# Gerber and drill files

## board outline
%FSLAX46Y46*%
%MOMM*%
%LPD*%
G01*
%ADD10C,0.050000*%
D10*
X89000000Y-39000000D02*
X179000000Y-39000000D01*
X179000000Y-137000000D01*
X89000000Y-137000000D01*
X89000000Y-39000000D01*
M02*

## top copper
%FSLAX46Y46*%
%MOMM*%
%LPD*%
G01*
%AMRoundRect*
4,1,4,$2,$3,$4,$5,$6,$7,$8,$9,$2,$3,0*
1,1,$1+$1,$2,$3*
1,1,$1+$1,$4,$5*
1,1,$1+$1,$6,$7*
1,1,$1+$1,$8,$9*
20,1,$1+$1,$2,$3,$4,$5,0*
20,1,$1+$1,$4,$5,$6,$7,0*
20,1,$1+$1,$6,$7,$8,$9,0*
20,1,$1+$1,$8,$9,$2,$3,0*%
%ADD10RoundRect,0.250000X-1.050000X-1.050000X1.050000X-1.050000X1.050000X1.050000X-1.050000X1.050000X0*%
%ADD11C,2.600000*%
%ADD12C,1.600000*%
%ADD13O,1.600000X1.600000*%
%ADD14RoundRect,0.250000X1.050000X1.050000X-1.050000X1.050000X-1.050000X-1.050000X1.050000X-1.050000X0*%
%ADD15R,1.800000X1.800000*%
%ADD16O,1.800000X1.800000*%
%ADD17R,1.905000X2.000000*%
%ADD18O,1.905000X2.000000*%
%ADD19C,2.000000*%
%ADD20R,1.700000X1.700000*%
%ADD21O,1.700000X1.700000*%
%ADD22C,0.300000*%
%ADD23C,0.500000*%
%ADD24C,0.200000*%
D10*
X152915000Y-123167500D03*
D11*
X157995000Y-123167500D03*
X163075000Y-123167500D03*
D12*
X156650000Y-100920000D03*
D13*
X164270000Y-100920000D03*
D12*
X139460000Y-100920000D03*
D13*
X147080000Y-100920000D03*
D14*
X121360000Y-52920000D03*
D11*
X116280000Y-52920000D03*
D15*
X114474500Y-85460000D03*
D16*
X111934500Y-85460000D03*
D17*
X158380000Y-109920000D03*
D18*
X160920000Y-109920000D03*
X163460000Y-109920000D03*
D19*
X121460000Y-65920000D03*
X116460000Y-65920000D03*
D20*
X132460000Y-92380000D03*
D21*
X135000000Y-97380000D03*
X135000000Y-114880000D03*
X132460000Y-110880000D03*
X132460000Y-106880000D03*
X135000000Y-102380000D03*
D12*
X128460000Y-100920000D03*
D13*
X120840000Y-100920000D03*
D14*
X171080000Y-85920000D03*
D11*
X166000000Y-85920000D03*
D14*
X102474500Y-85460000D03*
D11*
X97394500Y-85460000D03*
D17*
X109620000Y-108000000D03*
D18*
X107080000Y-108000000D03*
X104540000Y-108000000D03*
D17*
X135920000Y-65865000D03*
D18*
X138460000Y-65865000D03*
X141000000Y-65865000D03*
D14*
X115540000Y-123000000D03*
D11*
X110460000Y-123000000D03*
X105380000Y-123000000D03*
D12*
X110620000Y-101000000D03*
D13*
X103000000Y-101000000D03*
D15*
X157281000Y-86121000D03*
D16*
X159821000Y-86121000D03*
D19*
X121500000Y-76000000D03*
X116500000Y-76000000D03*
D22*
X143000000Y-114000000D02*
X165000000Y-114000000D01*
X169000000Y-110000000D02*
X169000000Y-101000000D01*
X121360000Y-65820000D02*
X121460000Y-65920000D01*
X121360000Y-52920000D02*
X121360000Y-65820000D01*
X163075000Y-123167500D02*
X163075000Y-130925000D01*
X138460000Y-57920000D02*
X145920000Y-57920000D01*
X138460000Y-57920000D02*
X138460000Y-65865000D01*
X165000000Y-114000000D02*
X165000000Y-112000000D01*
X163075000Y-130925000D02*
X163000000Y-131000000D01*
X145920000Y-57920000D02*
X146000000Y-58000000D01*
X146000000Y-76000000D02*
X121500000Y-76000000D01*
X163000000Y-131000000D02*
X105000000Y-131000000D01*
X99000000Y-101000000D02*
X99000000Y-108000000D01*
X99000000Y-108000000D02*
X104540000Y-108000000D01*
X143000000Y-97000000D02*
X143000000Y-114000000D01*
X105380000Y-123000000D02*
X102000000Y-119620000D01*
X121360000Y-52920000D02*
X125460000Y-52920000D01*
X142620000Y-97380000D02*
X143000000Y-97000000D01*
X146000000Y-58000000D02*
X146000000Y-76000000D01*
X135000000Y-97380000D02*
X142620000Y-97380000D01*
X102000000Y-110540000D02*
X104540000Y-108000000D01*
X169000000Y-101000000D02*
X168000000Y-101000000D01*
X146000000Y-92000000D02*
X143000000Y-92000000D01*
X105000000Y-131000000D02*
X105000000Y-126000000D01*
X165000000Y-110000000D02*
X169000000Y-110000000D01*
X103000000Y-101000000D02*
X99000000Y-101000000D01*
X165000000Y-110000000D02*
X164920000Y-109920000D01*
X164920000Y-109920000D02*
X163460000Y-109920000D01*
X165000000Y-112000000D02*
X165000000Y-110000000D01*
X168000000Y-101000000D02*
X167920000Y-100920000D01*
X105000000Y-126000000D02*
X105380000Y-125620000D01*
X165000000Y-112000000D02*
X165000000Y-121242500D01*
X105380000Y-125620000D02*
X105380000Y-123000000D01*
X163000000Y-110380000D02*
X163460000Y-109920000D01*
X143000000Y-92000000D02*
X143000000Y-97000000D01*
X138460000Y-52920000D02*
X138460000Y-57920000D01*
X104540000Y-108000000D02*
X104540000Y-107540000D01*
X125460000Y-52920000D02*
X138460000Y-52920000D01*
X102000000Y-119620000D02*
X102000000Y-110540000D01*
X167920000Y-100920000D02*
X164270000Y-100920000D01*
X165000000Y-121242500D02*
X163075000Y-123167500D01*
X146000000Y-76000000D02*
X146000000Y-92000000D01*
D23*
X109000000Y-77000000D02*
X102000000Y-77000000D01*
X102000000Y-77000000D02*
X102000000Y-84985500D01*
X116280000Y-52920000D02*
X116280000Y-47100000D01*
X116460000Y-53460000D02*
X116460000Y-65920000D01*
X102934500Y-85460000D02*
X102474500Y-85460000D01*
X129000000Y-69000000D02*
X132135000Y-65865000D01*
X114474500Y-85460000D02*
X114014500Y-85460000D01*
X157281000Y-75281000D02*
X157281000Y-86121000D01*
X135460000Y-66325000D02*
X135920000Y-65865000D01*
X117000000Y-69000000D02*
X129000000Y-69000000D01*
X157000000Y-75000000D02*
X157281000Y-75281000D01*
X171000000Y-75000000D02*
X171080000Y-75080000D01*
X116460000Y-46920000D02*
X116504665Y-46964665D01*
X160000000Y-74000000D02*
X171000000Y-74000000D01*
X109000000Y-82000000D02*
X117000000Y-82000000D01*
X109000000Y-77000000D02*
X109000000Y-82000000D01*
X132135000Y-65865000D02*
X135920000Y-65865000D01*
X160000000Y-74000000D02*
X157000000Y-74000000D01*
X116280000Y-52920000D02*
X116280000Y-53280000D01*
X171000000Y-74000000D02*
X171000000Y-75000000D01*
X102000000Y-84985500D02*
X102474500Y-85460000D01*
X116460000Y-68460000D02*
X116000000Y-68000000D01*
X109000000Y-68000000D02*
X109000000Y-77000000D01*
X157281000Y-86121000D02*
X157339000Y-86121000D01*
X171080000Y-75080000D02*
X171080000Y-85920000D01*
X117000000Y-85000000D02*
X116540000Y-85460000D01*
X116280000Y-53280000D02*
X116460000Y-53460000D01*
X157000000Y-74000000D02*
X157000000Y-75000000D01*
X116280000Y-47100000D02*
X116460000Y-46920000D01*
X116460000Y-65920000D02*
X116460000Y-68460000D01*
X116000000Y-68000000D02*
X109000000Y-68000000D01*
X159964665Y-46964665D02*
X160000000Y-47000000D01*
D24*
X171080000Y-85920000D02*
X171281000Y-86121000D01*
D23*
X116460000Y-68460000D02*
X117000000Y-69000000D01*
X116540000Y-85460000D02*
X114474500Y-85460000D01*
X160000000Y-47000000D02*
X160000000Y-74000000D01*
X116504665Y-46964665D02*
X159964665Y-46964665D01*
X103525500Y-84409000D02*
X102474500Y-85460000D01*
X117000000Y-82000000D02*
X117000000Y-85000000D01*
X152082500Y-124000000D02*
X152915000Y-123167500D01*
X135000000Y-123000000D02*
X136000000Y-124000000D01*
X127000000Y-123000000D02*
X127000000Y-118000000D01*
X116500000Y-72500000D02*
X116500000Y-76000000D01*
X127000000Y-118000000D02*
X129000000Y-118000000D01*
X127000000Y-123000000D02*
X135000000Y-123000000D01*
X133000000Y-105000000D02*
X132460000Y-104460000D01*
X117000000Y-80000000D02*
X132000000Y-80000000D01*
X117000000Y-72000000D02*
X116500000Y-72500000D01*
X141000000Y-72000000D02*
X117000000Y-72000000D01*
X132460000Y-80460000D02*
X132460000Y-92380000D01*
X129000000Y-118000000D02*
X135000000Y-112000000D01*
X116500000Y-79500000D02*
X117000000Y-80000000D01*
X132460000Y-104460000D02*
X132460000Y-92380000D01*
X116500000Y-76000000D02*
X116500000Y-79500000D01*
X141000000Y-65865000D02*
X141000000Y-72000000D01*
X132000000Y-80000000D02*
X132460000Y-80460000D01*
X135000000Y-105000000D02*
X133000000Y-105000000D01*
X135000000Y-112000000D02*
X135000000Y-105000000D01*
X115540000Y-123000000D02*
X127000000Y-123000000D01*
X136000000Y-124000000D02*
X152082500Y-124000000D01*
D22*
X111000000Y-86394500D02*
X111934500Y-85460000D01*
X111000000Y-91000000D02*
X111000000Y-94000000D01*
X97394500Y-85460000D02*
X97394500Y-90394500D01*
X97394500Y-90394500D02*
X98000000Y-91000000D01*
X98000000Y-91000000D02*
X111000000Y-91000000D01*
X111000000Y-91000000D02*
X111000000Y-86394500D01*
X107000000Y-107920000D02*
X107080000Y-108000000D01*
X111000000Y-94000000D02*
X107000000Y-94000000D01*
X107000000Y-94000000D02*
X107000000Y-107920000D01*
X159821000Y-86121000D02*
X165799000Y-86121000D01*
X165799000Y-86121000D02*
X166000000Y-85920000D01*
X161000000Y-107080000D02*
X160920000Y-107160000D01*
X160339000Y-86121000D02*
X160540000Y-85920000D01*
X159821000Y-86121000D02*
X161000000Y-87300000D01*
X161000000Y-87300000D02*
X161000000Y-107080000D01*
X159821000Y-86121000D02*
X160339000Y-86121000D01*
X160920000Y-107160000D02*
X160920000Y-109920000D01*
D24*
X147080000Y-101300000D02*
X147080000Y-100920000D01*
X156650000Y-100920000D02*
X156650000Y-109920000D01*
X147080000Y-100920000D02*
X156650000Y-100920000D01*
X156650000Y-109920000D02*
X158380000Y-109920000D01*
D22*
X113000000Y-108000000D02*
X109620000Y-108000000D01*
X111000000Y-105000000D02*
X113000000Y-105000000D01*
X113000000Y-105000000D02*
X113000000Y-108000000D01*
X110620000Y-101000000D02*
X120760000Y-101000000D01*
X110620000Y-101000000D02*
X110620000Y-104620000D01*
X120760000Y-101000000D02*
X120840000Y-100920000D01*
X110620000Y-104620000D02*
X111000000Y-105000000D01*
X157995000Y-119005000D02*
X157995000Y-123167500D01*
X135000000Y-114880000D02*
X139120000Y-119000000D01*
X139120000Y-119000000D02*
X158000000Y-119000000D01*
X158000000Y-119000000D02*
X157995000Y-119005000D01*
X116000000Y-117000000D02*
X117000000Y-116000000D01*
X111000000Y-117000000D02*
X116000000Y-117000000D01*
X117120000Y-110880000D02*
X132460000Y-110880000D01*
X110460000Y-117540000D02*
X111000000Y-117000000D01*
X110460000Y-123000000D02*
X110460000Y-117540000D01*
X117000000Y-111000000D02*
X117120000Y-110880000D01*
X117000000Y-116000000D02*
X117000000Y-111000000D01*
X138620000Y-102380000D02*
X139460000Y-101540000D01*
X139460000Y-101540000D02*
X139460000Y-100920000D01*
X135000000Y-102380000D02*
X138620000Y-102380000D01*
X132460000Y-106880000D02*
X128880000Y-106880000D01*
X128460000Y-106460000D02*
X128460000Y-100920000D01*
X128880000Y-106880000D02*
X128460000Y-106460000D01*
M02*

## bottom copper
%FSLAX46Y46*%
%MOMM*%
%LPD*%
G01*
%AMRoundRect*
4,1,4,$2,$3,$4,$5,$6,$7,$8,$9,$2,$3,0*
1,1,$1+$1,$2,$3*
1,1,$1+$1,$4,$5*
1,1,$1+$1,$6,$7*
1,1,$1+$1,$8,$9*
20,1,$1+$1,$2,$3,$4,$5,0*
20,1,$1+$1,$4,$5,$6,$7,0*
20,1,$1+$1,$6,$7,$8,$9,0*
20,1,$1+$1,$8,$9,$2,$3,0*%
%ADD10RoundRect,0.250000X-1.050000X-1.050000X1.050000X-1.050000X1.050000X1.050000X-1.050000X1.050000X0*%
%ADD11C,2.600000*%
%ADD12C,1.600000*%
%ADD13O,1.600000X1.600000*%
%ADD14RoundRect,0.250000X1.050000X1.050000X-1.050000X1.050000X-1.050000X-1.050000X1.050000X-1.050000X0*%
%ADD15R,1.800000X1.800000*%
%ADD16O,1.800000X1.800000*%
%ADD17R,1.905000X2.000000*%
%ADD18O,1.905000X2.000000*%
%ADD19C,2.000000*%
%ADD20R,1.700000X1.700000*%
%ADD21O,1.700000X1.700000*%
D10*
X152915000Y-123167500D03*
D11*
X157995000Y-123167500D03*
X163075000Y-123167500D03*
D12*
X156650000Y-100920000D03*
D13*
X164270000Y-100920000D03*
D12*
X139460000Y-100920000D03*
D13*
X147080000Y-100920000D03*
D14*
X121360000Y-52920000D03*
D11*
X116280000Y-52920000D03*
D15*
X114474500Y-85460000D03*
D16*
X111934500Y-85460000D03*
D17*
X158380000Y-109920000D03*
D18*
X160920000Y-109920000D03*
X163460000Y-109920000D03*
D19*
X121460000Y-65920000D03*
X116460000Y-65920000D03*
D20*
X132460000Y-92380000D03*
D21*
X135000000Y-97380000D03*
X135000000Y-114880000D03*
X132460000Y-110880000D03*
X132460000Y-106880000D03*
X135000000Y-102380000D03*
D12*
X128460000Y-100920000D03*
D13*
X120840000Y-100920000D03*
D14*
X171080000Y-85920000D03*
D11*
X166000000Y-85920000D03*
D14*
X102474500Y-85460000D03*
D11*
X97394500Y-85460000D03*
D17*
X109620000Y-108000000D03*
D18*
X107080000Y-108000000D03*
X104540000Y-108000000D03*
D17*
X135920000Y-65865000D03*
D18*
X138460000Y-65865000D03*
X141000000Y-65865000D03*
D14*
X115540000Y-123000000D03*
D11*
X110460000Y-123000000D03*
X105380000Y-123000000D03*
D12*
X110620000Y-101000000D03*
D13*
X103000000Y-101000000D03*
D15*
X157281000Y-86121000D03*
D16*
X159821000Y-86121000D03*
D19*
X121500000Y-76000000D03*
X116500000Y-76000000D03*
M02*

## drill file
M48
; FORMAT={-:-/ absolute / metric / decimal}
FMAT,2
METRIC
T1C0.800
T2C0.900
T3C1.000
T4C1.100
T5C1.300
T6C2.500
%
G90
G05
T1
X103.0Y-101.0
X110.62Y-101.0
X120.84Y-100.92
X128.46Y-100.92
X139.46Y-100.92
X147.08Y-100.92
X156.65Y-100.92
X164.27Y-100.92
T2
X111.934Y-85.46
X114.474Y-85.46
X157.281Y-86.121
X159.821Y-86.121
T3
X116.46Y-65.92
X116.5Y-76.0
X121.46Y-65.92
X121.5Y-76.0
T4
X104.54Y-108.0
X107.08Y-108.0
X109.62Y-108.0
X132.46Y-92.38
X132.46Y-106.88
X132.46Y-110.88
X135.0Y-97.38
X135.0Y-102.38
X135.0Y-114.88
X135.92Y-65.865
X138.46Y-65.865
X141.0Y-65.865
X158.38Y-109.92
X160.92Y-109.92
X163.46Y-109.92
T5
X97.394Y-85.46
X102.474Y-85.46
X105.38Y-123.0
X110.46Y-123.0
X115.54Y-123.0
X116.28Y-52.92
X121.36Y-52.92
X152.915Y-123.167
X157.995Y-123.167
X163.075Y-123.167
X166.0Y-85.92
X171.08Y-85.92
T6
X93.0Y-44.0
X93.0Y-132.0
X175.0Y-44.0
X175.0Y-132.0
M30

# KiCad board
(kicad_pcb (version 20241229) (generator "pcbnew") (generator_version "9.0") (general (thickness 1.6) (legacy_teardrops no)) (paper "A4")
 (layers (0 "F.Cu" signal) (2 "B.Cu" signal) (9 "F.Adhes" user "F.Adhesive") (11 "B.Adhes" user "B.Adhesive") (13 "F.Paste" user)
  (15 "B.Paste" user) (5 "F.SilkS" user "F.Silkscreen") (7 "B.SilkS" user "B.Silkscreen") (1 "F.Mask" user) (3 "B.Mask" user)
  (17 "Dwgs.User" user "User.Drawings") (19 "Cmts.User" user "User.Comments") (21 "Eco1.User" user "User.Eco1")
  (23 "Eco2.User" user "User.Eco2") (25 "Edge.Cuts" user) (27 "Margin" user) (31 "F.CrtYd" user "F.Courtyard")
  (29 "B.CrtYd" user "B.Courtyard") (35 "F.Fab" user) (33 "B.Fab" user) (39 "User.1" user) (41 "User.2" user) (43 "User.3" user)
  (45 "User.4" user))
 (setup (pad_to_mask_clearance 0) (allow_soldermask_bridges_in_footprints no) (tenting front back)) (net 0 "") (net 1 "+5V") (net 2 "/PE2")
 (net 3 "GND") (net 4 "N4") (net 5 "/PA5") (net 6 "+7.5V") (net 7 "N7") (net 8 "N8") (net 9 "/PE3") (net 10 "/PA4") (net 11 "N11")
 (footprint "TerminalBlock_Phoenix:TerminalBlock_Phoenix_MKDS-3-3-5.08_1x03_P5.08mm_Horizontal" (layer "F.Cu") (at 152.915 123.1675)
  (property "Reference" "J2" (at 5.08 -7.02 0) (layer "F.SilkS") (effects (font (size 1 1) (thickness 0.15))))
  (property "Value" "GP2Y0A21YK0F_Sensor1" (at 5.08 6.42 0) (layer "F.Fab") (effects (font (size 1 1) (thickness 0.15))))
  (pad "1" thru_hole roundrect (at 0 0) (size 2.6 2.6) (drill 1.3) (layers "*.Cu" "*.Mask") (remove_unused_layers no)
   (roundrect_rratio 0.096154) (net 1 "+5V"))
  (pad "2" thru_hole circle (at 5.08 0) (size 2.6 2.6) (drill 1.3) (layers "*.Cu" "*.Mask") (remove_unused_layers no) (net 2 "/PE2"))
  (pad "3" thru_hole circle (at 10.16 0) (size 2.6 2.6) (drill 1.3) (layers "*.Cu" "*.Mask") (remove_unused_layers no) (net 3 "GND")))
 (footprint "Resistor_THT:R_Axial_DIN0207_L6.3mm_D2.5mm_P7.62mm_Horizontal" (layer "F.Cu") (at 156.65 100.92)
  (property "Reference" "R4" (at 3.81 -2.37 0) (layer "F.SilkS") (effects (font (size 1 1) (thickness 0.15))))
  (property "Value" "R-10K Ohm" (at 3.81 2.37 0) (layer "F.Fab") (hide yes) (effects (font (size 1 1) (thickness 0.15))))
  (pad "1" thru_hole circle (at 0 0) (size 1.6 1.6) (drill 0.8) (layers "*.Cu" "*.Mask") (remove_unused_layers no) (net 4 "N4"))
  (pad "2" thru_hole oval (at 7.62 0) (size 1.6 1.6) (drill 0.8) (layers "*.Cu" "*.Mask") (remove_unused_layers no) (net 3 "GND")))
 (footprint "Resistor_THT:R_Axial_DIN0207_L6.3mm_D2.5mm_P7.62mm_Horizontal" (layer "F.Cu") (at 139.46 100.92)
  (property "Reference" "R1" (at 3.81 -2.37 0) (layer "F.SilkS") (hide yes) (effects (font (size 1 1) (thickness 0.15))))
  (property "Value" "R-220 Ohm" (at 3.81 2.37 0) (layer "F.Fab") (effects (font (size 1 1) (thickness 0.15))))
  (pad "1" thru_hole circle (at 0 0) (size 1.6 1.6) (drill 0.8) (layers "*.Cu" "*.Mask") (remove_unused_layers no) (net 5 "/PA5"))
  (pad "2" thru_hole oval (at 7.62 0) (size 1.6 1.6) (drill 0.8) (layers "*.Cu" "*.Mask") (remove_unused_layers no) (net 4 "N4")))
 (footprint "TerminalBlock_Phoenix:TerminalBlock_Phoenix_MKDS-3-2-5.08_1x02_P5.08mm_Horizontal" (layer "F.Cu") (at 121.36 52.92 180)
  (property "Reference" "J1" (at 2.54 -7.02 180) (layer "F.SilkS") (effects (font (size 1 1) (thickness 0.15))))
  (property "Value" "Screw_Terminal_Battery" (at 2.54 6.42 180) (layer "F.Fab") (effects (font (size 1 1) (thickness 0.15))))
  (pad "1" thru_hole roundrect (at 0 0 180) (size 2.6 2.6) (drill 1.3) (layers "*.Cu" "*.Mask") (remove_unused_layers no)
   (roundrect_rratio 0.096154) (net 3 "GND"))
  (pad "2" thru_hole circle (at 5.08 0 180) (size 2.6 2.6) (drill 1.3) (layers "*.Cu" "*.Mask") (remove_unused_layers no) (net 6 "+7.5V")))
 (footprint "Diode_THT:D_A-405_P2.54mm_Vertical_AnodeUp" (layer "F.Cu") (at 114.4745 85.46 180)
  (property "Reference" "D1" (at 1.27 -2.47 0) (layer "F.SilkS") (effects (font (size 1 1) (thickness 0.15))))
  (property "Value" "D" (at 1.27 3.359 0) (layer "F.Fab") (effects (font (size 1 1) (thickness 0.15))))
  (pad "1" thru_hole rect (at 0 0 180) (size 1.8 1.8) (drill 0.9) (layers "*.Cu" "*.Mask") (remove_unused_layers no) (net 6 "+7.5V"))
  (pad "2" thru_hole oval (at 2.54 0 180) (size 1.8 1.8) (drill 0.9) (layers "*.Cu" "*.Mask") (remove_unused_layers no) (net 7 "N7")))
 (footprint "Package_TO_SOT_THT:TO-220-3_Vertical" (layer "F.Cu") (at 158.38 109.92)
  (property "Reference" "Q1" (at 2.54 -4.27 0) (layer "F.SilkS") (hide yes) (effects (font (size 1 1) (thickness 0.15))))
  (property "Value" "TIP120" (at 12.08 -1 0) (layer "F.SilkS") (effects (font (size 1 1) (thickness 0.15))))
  (pad "1" thru_hole rect (at 0 0) (size 1.905 2) (drill 1.1) (layers "*.Cu" "*.Mask") (remove_unused_layers no) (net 4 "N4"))
  (pad "2" thru_hole oval (at 2.54 0) (size 1.905 2) (drill 1.1) (layers "*.Cu" "*.Mask") (remove_unused_layers no) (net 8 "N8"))
  (pad "3" thru_hole oval (at 5.08 0) (size 1.905 2) (drill 1.1) (layers "*.Cu" "*.Mask") (remove_unused_layers no) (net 3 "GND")))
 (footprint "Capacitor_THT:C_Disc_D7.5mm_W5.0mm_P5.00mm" (layer "F.Cu") (at 121.46 65.92 180)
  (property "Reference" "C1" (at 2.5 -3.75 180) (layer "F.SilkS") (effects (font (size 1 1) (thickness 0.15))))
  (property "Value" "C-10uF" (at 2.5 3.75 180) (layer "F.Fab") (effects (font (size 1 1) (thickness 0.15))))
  (pad "1" thru_hole circle (at 0 0 180) (size 2 2) (drill 1) (layers "*.Cu" "*.Mask") (remove_unused_layers no) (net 3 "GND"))
  (pad "2" thru_hole circle (at 5 0 180) (size 2 2) (drill 1) (layers "*.Cu" "*.Mask") (remove_unused_layers no) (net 6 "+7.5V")))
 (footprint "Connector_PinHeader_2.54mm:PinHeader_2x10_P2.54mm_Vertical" (layer "F.Cu") (at 132.46 92.38)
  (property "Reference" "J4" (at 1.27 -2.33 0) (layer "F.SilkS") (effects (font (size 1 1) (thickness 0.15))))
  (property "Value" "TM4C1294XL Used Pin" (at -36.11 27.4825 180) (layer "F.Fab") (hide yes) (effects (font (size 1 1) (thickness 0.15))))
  (pad "1" thru_hole rect (at 0 0) (size 1.7 1.7) (drill 1.1) (layers "*.Cu" "*.Mask") (remove_unused_layers no) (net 1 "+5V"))
  (pad "2" thru_hole oval (at 2.54 5) (size 1.7 1.7) (drill 1.1) (layers "*.Cu" "*.Mask") (remove_unused_layers no) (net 3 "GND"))
  (pad "4" thru_hole oval (at 2.54 22.5) (size 1.7 1.7) (drill 1.1) (layers "*.Cu" "*.Mask") (remove_unused_layers no) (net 2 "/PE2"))
  (pad "5" thru_hole oval (at 0 18.5) (size 1.7 1.7) (drill 1.1) (layers "*.Cu" "*.Mask") (remove_unused_layers no) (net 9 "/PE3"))
  (pad "7" thru_hole oval (at 0 14.5) (size 1.7 1.7) (drill 1.1) (layers "*.Cu" "*.Mask") (remove_unused_layers no) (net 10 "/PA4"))
  (pad "8" thru_hole oval (at 2.54 10) (size 1.7 1.7) (drill 1.1) (layers "*.Cu" "*.Mask") (remove_unused_layers no) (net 5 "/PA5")))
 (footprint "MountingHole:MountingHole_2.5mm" (layer "F.Cu") (at 93 44)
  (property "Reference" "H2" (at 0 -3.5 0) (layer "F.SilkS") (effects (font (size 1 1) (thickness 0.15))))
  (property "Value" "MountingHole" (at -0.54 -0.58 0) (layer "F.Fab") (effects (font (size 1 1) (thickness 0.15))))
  (pad "" np_thru_hole circle (at 0 0) (size 2.5 2.5) (drill 2.5) (layers "*.Cu" "*.Mask")))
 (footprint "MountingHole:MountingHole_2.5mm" (layer "F.Cu") (at 93 132)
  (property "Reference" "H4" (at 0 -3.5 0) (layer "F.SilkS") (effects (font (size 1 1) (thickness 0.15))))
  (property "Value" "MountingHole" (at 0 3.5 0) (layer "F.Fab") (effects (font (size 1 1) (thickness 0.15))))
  (pad "" np_thru_hole circle (at 0 0) (size 2.5 2.5) (drill 2.5) (layers "*.Cu" "*.Mask")))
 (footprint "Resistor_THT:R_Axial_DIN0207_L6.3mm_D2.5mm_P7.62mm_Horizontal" (layer "F.Cu") (at 128.46 100.92 180)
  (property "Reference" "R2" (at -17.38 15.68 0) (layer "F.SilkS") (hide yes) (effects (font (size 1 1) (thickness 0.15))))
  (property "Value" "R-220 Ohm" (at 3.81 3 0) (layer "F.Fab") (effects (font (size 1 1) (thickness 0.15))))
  (pad "1" thru_hole circle (at 0 0 180) (size 1.6 1.6) (drill 0.8) (layers "*.Cu" "*.Mask") (remove_unused_layers no) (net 10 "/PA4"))
  (pad "2" thru_hole oval (at 7.62 0 180) (size 1.6 1.6) (drill 0.8) (layers "*.Cu" "*.Mask") (remove_unused_layers no) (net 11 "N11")))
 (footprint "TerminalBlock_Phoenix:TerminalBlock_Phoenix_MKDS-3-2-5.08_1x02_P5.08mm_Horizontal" (layer "F.Cu") (at 171.08 85.92 180)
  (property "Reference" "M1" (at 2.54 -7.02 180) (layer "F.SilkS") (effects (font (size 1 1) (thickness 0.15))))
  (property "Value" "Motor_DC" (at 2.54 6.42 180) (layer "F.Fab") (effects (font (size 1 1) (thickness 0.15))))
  (pad "1" thru_hole roundrect (at 0 0 180) (size 2.6 2.6) (drill 1.3) (layers "*.Cu" "*.Mask") (remove_unused_layers no)
   (roundrect_rratio 0.096154) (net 6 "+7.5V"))
  (pad "2" thru_hole circle (at 5.08 0 180) (size 2.6 2.6) (drill 1.3) (layers "*.Cu" "*.Mask") (remove_unused_layers no) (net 8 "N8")))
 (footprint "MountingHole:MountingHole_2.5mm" (layer "F.Cu") (at 175 132)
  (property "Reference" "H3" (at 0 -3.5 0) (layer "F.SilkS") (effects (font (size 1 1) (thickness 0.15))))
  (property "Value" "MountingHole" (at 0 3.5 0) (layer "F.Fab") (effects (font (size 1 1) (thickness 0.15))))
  (pad "" np_thru_hole circle (at 0 0) (size 2.5 2.5) (drill 2.5) (layers "*.Cu" "*.Mask")))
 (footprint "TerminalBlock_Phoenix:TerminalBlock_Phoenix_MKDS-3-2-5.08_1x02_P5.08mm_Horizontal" (layer "F.Cu") (at 102.4745 85.46 180)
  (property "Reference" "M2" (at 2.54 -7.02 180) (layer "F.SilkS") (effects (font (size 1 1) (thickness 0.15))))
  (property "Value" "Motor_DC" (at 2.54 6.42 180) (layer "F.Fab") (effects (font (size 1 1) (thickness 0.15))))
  (pad "1" thru_hole roundrect (at 0 0 180) (size 2.6 2.6) (drill 1.3) (layers "*.Cu" "*.Mask") (remove_unused_layers no)
   (roundrect_rratio 0.096154) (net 6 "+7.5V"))
  (pad "2" thru_hole circle (at 5.08 0 180) (size 2.6 2.6) (drill 1.3) (layers "*.Cu" "*.Mask") (remove_unused_layers no) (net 7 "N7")))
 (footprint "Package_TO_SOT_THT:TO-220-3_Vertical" (layer "F.Cu") (at 109.62 108 180)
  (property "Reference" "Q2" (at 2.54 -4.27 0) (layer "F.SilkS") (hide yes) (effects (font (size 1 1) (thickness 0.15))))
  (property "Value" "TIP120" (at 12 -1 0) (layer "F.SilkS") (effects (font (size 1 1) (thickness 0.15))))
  (pad "1" thru_hole rect (at 0 0 180) (size 1.905 2) (drill 1.1) (layers "*.Cu" "*.Mask") (remove_unused_layers no) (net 11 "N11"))
  (pad "2" thru_hole oval (at 2.54 0 180) (size 1.905 2) (drill 1.1) (layers "*.Cu" "*.Mask") (remove_unused_layers no) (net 7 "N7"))
  (pad "3" thru_hole oval (at 5.08 0 180) (size 1.905 2) (drill 1.1) (layers "*.Cu" "*.Mask") (remove_unused_layers no) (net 3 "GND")))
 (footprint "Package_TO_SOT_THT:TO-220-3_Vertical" (layer "F.Cu") (at 135.92 65.865)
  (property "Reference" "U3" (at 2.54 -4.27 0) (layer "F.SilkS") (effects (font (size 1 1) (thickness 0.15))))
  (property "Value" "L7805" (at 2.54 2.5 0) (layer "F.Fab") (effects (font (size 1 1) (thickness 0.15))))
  (pad "1" thru_hole rect (at 0 0) (size 1.905 2) (drill 1.1) (layers "*.Cu" "*.Mask") (remove_unused_layers no) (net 6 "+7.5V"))
  (pad "2" thru_hole oval (at 2.54 0) (size 1.905 2) (drill 1.1) (layers "*.Cu" "*.Mask") (remove_unused_layers no) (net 3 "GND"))
  (pad "3" thru_hole oval (at 5.08 0) (size 1.905 2) (drill 1.1) (layers "*.Cu" "*.Mask") (remove_unused_layers no) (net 1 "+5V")))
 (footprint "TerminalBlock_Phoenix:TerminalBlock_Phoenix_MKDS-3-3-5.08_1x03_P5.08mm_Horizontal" (layer "F.Cu") (at 115.54 123 180)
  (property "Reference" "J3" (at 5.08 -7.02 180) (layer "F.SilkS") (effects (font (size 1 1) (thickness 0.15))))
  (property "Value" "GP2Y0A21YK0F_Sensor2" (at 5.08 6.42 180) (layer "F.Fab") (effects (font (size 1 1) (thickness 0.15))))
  (pad "1" thru_hole roundrect (at 0 0 180) (size 2.6 2.6) (drill 1.3) (layers "*.Cu" "*.Mask") (remove_unused_layers no)
   (roundrect_rratio 0.096154) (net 1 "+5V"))
  (pad "2" thru_hole circle (at 5.08 0 180) (size 2.6 2.6) (drill 1.3) (layers "*.Cu" "*.Mask") (remove_unused_layers no) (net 9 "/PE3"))
  (pad "3" thru_hole circle (at 10.16 0 180) (size 2.6 2.6) (drill 1.3) (layers "*.Cu" "*.Mask") (remove_unused_layers no) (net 3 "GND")))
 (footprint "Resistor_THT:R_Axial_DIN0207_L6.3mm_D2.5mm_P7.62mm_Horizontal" (layer "F.Cu") (at 110.62 101 180)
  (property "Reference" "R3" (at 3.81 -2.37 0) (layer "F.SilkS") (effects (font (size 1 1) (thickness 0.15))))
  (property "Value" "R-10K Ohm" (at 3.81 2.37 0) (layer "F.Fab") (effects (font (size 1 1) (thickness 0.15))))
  (pad "1" thru_hole circle (at 0 0 180) (size 1.6 1.6) (drill 0.8) (layers "*.Cu" "*.Mask") (remove_unused_layers no) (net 11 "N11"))
  (pad "2" thru_hole oval (at 7.62 0 180) (size 1.6 1.6) (drill 0.8) (layers "*.Cu" "*.Mask") (remove_unused_layers no) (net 3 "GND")))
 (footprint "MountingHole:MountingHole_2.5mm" (layer "F.Cu") (at 175 44)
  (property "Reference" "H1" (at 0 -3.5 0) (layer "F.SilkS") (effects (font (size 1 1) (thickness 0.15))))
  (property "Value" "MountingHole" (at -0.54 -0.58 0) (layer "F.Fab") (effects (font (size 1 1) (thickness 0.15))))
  (pad "" np_thru_hole circle (at 0 0) (size 2.5 2.5) (drill 2.5) (layers "*.Cu" "*.Mask")))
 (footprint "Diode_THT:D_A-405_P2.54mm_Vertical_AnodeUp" (layer "F.Cu") (at 157.281 86.121)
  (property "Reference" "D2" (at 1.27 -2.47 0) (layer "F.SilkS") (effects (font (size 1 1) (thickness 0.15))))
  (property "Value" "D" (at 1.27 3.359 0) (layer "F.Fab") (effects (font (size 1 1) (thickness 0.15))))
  (pad "1" thru_hole rect (at 0 0) (size 1.8 1.8) (drill 0.9) (layers "*.Cu" "*.Mask") (remove_unused_layers no) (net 6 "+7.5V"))
  (pad "2" thru_hole oval (at 2.54 0) (size 1.8 1.8) (drill 0.9) (layers "*.Cu" "*.Mask") (remove_unused_layers no) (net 8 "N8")))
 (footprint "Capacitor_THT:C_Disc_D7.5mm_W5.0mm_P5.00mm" (layer "F.Cu") (at 121.5 76 180)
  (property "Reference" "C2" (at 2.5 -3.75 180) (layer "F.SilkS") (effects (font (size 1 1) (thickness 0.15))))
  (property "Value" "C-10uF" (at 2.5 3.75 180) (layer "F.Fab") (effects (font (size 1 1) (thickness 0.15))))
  (pad "1" thru_hole circle (at 0 0 180) (size 2 2) (drill 1) (layers "*.Cu" "*.Mask") (remove_unused_layers no) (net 3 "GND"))
  (pad "2" thru_hole circle (at 5 0 180) (size 2 2) (drill 1) (layers "*.Cu" "*.Mask") (remove_unused_layers no) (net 1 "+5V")))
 (gr_rect (start 89 39) (end 179 137) (stroke (width 0.05) (type default)) (fill no) (layer "Edge.Cuts"))
 (segment (start 143 114) (end 165 114) (width 0.3) (layer "F.Cu") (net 3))
 (segment (start 169 110) (end 169 101) (width 0.3) (layer "F.Cu") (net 3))
 (segment (start 121.36 65.82) (end 121.46 65.92) (width 0.3) (layer "F.Cu") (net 3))
 (segment (start 121.36 52.92) (end 121.36 65.82) (width 0.3) (layer "F.Cu") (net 3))
 (segment (start 163.075 123.1675) (end 163.075 130.925) (width 0.3) (layer "F.Cu") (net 3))
 (segment (start 138.46 57.92) (end 145.92 57.92) (width 0.3) (layer "F.Cu") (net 3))
 (segment (start 138.46 57.92) (end 138.46 65.865) (width 0.3) (layer "F.Cu") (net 3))
 (segment (start 165 114) (end 165 112) (width 0.3) (layer "F.Cu") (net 3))
 (segment (start 163.075 130.925) (end 163 131) (width 0.3) (layer "F.Cu") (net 3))
 (segment (start 145.92 57.92) (end 146 58) (width 0.3) (layer "F.Cu") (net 3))
 (segment (start 146 76) (end 121.5 76) (width 0.3) (layer "F.Cu") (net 3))
 (segment (start 163 131) (end 105 131) (width 0.3) (layer "F.Cu") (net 3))
 (segment (start 99 101) (end 99 108) (width 0.3) (layer "F.Cu") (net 3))
 (segment (start 99 108) (end 104.54 108) (width 0.3) (layer "F.Cu") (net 3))
 (segment (start 143 97) (end 143 114) (width 0.3) (layer "F.Cu") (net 3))
 (segment (start 105.38 123) (end 102 119.62) (width 0.3) (layer "F.Cu") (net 3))
 (segment (start 121.36 52.92) (end 125.46 52.92) (width 0.3) (layer "F.Cu") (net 3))
 (segment (start 142.62 97.38) (end 143 97) (width 0.3) (layer "F.Cu") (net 3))
 (segment (start 146 58) (end 146 76) (width 0.3) (layer "F.Cu") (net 3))
 (segment (start 135 97.38) (end 142.62 97.38) (width 0.3) (layer "F.Cu") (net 3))
 (segment (start 102 110.54) (end 104.54 108) (width 0.3) (layer "F.Cu") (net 3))
 (segment (start 169 101) (end 168 101) (width 0.3) (layer "F.Cu") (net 3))
 (segment (start 146 92) (end 143 92) (width 0.3) (layer "F.Cu") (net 3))
 (segment (start 105 131) (end 105 126) (width 0.3) (layer "F.Cu") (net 3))
 (segment (start 165 110) (end 169 110) (width 0.3) (layer "F.Cu") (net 3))
 (segment (start 103 101) (end 99 101) (width 0.3) (layer "F.Cu") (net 3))
 (segment (start 165 110) (end 164.92 109.92) (width 0.3) (layer "F.Cu") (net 3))
 (segment (start 164.92 109.92) (end 163.46 109.92) (width 0.3) (layer "F.Cu") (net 3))
 (segment (start 165 112) (end 165 110) (width 0.3) (layer "F.Cu") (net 3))
 (segment (start 168 101) (end 167.92 100.92) (width 0.3) (layer "F.Cu") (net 3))
 (segment (start 105 126) (end 105.38 125.62) (width 0.3) (layer "F.Cu") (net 3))
 (segment (start 165 112) (end 165 121.2425) (width 0.3) (layer "F.Cu") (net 3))
 (segment (start 105.38 125.62) (end 105.38 123) (width 0.3) (layer "F.Cu") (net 3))
 (segment (start 163 110.38) (end 163.46 109.92) (width 0.3) (layer "F.Cu") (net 3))
 (segment (start 143 92) (end 143 97) (width 0.3) (layer "F.Cu") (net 3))
 (segment (start 138.46 52.92) (end 138.46 57.92) (width 0.3) (layer "F.Cu") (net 3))
 (segment (start 104.54 108) (end 104.54 107.54) (width 0.3) (layer "F.Cu") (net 3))
 (segment (start 125.46 52.92) (end 138.46 52.92) (width 0.3) (layer "F.Cu") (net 3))
 (segment (start 102 119.62) (end 102 110.54) (width 0.3) (layer "F.Cu") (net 3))
 (segment (start 167.92 100.92) (end 164.27 100.92) (width 0.3) (layer "F.Cu") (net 3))
 (segment (start 165 121.2425) (end 163.075 123.1675) (width 0.3) (layer "F.Cu") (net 3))
 (segment (start 146 76) (end 146 92) (width 0.3) (layer "F.Cu") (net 3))
 (segment (start 109 77) (end 102 77) (width 0.5) (layer "F.Cu") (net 6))
 (segment (start 102 77) (end 102 84.9855) (width 0.5) (layer "F.Cu") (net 6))
 (segment (start 116.28 52.92) (end 116.28 47.1) (width 0.5) (layer "F.Cu") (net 6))
 (segment (start 116.46 53.46) (end 116.46 65.92) (width 0.5) (layer "F.Cu") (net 6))
 (segment (start 102.9345 85.46) (end 102.4745 85.46) (width 0.5) (layer "F.Cu") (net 6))
 (segment (start 129 69) (end 132.135 65.865) (width 0.5) (layer "F.Cu") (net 6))
 (segment (start 114.4745 85.46) (end 114.0145 85.46) (width 0.5) (layer "F.Cu") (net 6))
 (segment (start 157.281 75.281) (end 157.281 86.121) (width 0.5) (layer "F.Cu") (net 6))
 (segment (start 135.46 66.325) (end 135.92 65.865) (width 0.5) (layer "F.Cu") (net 6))
 (segment (start 117 69) (end 129 69) (width 0.5) (layer "F.Cu") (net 6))
 (segment (start 157 75) (end 157.281 75.281) (width 0.5) (layer "F.Cu") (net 6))
 (segment (start 171 75) (end 171.08 75.08) (width 0.5) (layer "F.Cu") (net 6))
 (segment (start 116.46 46.92) (end 116.504665 46.964665) (width 0.5) (layer "F.Cu") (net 6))
 (segment (start 160 74) (end 171 74) (width 0.5) (layer "F.Cu") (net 6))
 (segment (start 109 82) (end 117 82) (width 0.5) (layer "F.Cu") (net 6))
 (segment (start 109 77) (end 109 82) (width 0.5) (layer "F.Cu") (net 6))
 (segment (start 132.135 65.865) (end 135.92 65.865) (width 0.5) (layer "F.Cu") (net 6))
 (segment (start 160 74) (end 157 74) (width 0.5) (layer "F.Cu") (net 6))
 (segment (start 116.28 52.92) (end 116.28 53.28) (width 0.5) (layer "F.Cu") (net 6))
 (segment (start 171 74) (end 171 75) (width 0.5) (layer "F.Cu") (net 6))
 (segment (start 102 84.9855) (end 102.4745 85.46) (width 0.5) (layer "F.Cu") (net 6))
 (segment (start 116.46 68.46) (end 116 68) (width 0.5) (layer "F.Cu") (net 6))
 (segment (start 109 68) (end 109 77) (width 0.5) (layer "F.Cu") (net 6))
 (segment (start 157.281 86.121) (end 157.339 86.121) (width 0.5) (layer "F.Cu") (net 6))
 (segment (start 171.08 75.08) (end 171.08 85.92) (width 0.5) (layer "F.Cu") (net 6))
 (segment (start 117 85) (end 116.54 85.46) (width 0.5) (layer "F.Cu") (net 6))
 (segment (start 116.28 53.28) (end 116.46 53.46) (width 0.5) (layer "F.Cu") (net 6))
 (segment (start 157 74) (end 157 75) (width 0.5) (layer "F.Cu") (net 6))
 (segment (start 116.28 47.1) (end 116.46 46.92) (width 0.5) (layer "F.Cu") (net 6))
 (segment (start 116.46 65.92) (end 116.46 68.46) (width 0.5) (layer "F.Cu") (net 6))
 (segment (start 116 68) (end 109 68) (width 0.5) (layer "F.Cu") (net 6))
 (segment (start 159.964665 46.964665) (end 160 47) (width 0.5) (layer "F.Cu") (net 6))
 (segment (start 171.08 85.92) (end 171.281 86.121) (width 0.2) (layer "F.Cu") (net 6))
 (segment (start 116.46 68.46) (end 117 69) (width 0.5) (layer "F.Cu") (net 6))
 (segment (start 116.54 85.46) (end 114.4745 85.46) (width 0.5) (layer "F.Cu") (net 6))
 (segment (start 160 47) (end 160 74) (width 0.5) (layer "F.Cu") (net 6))
 (segment (start 116.504665 46.964665) (end 159.964665 46.964665) (width 0.5) (layer "F.Cu") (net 6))
 (segment (start 103.5255 84.409) (end 102.4745 85.46) (width 0.5) (layer "F.Cu") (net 6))
 (segment (start 117 82) (end 117 85) (width 0.5) (layer "F.Cu") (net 6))
 (segment (start 152.0825 124) (end 152.915 123.1675) (width 0.5) (layer "F.Cu") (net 1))
 (segment (start 135 123) (end 136 124) (width 0.5) (layer "F.Cu") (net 1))
 (segment (start 127 123) (end 127 118) (width 0.5) (layer "F.Cu") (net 1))
 (segment (start 116.5 72.5) (end 116.5 76) (width 0.5) (layer "F.Cu") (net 1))
 (segment (start 127 118) (end 129 118) (width 0.5) (layer "F.Cu") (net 1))
 (segment (start 127 123) (end 135 123) (width 0.5) (layer "F.Cu") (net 1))
 (segment (start 133 105) (end 132.46 104.46) (width 0.5) (layer "F.Cu") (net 1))
 (segment (start 117 80) (end 132 80) (width 0.5) (layer "F.Cu") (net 1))
 (segment (start 117 72) (end 116.5 72.5) (width 0.5) (layer "F.Cu") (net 1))
 (segment (start 141 72) (end 117 72) (width 0.5) (layer "F.Cu") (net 1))
 (segment (start 132.46 80.46) (end 132.46 92.38) (width 0.5) (layer "F.Cu") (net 1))
 (segment (start 129 118) (end 135 112) (width 0.5) (layer "F.Cu") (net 1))
 (segment (start 116.5 79.5) (end 117 80) (width 0.5) (layer "F.Cu") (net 1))
 (segment (start 132.46 104.46) (end 132.46 92.38) (width 0.5) (layer "F.Cu") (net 1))
 (segment (start 116.5 76) (end 116.5 79.5) (width 0.5) (layer "F.Cu") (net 1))
 (segment (start 141 65.865) (end 141 72) (width 0.5) (layer "F.Cu") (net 1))
 (segment (start 132 80) (end 132.46 80.46) (width 0.5) (layer "F.Cu") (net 1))
 (segment (start 135 105) (end 133 105) (width 0.5) (layer "F.Cu") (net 1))
 (segment (start 135 112) (end 135 105) (width 0.5) (layer "F.Cu") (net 1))
 (segment (start 115.54 123) (end 127 123) (width 0.5) (layer "F.Cu") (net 1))
 (segment (start 136 124) (end 152.0825 124) (width 0.5) (layer "F.Cu") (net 1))
 (segment (start 111 86.3945) (end 111.9345 85.46) (width 0.3) (layer "F.Cu") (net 7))
 (segment (start 111 91) (end 111 94) (width 0.3) (layer "F.Cu") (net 7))
 (segment (start 97.3945 85.46) (end 97.3945 90.3945) (width 0.3) (layer "F.Cu") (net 7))
 (segment (start 97.3945 90.3945) (end 98 91) (width 0.3) (layer "F.Cu") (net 7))
 (segment (start 98 91) (end 111 91) (width 0.3) (layer "F.Cu") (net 7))
 (segment (start 111 91) (end 111 86.3945) (width 0.3) (layer "F.Cu") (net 7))
 (segment (start 107 107.92) (end 107.08 108) (width 0.3) (layer "F.Cu") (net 7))
 (segment (start 111 94) (end 107 94) (width 0.3) (layer "F.Cu") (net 7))
 (segment (start 107 94) (end 107 107.92) (width 0.3) (layer "F.Cu") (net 7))
 (segment (start 159.821 86.121) (end 165.799 86.121) (width 0.3) (layer "F.Cu") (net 8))
 (segment (start 165.799 86.121) (end 166 85.92) (width 0.3) (layer "F.Cu") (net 8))
 (segment (start 161 107.08) (end 160.92 107.16) (width 0.3) (layer "F.Cu") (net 8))
 (segment (start 160.339 86.121) (end 160.54 85.92) (width 0.3) (layer "F.Cu") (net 8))
 (segment (start 159.821 86.121) (end 161 87.3) (width 0.3) (layer "F.Cu") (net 8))
 (segment (start 161 87.3) (end 161 107.08) (width 0.3) (layer "F.Cu") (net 8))
 (segment (start 159.821 86.121) (end 160.339 86.121) (width 0.3) (layer "F.Cu") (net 8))
 (segment (start 160.92 107.16) (end 160.92 109.92) (width 0.3) (layer "F.Cu") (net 8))
 (segment (start 147.08 101.3) (end 147.08 100.92) (width 0.2) (layer "F.Cu") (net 4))
 (segment (start 156.65 100.92) (end 156.65 109.92) (width 0.2) (layer "F.Cu") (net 4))
 (segment (start 147.08 100.92) (end 156.65 100.92) (width 0.2) (layer "F.Cu") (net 4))
 (segment (start 156.65 109.92) (end 158.38 109.92) (width 0.2) (layer "F.Cu") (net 4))
 (segment (start 113 108) (end 109.62 108) (width 0.3) (layer "F.Cu") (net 11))
 (segment (start 111 105) (end 113 105) (width 0.3) (layer "F.Cu") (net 11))
 (segment (start 113 105) (end 113 108) (width 0.3) (layer "F.Cu") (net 11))
 (segment (start 110.62 101) (end 120.76 101) (width 0.3) (layer "F.Cu") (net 11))
 (segment (start 110.62 101) (end 110.62 104.62) (width 0.3) (layer "F.Cu") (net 11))
 (segment (start 120.76 101) (end 120.84 100.92) (width 0.3) (layer "F.Cu") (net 11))
 (segment (start 110.62 104.62) (end 111 105) (width 0.3) (layer "F.Cu") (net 11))
 (segment (start 157.995 119.005) (end 157.995 123.1675) (width 0.3) (layer "F.Cu") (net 2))
 (segment (start 135 114.88) (end 139.12 119) (width 0.3) (layer "F.Cu") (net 2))
 (segment (start 139.12 119) (end 158 119) (width 0.3) (layer "F.Cu") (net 2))
 (segment (start 158 119) (end 157.995 119.005) (width 0.3) (layer "F.Cu") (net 2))
 (segment (start 116 117) (end 117 116) (width 0.3) (layer "F.Cu") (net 9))
 (segment (start 111 117) (end 116 117) (width 0.3) (layer "F.Cu") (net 9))
 (segment (start 117.12 110.88) (end 132.46 110.88) (width 0.3) (layer "F.Cu") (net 9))
 (segment (start 110.46 117.54) (end 111 117) (width 0.3) (layer "F.Cu") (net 9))
 (segment (start 110.46 123) (end 110.46 117.54) (width 0.3) (layer "F.Cu") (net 9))
 (segment (start 117 111) (end 117.12 110.88) (width 0.3) (layer "F.Cu") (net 9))
 (segment (start 117 116) (end 117 111) (width 0.3) (layer "F.Cu") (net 9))
 (segment (start 138.62 102.38) (end 139.46 101.54) (width 0.3) (layer "F.Cu") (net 5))
 (segment (start 139.46 101.54) (end 139.46 100.92) (width 0.3) (layer "F.Cu") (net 5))
 (segment (start 135 102.38) (end 138.62 102.38) (width 0.3) (layer "F.Cu") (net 5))
 (segment (start 132.46 106.88) (end 128.88 106.88) (width 0.3) (layer "F.Cu") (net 10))
 (segment (start 128.46 106.46) (end 128.46 100.92) (width 0.3) (layer "F.Cu") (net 10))
 (segment (start 128.88 106.88) (end 128.46 106.46) (width 0.3) (layer "F.Cu") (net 10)))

